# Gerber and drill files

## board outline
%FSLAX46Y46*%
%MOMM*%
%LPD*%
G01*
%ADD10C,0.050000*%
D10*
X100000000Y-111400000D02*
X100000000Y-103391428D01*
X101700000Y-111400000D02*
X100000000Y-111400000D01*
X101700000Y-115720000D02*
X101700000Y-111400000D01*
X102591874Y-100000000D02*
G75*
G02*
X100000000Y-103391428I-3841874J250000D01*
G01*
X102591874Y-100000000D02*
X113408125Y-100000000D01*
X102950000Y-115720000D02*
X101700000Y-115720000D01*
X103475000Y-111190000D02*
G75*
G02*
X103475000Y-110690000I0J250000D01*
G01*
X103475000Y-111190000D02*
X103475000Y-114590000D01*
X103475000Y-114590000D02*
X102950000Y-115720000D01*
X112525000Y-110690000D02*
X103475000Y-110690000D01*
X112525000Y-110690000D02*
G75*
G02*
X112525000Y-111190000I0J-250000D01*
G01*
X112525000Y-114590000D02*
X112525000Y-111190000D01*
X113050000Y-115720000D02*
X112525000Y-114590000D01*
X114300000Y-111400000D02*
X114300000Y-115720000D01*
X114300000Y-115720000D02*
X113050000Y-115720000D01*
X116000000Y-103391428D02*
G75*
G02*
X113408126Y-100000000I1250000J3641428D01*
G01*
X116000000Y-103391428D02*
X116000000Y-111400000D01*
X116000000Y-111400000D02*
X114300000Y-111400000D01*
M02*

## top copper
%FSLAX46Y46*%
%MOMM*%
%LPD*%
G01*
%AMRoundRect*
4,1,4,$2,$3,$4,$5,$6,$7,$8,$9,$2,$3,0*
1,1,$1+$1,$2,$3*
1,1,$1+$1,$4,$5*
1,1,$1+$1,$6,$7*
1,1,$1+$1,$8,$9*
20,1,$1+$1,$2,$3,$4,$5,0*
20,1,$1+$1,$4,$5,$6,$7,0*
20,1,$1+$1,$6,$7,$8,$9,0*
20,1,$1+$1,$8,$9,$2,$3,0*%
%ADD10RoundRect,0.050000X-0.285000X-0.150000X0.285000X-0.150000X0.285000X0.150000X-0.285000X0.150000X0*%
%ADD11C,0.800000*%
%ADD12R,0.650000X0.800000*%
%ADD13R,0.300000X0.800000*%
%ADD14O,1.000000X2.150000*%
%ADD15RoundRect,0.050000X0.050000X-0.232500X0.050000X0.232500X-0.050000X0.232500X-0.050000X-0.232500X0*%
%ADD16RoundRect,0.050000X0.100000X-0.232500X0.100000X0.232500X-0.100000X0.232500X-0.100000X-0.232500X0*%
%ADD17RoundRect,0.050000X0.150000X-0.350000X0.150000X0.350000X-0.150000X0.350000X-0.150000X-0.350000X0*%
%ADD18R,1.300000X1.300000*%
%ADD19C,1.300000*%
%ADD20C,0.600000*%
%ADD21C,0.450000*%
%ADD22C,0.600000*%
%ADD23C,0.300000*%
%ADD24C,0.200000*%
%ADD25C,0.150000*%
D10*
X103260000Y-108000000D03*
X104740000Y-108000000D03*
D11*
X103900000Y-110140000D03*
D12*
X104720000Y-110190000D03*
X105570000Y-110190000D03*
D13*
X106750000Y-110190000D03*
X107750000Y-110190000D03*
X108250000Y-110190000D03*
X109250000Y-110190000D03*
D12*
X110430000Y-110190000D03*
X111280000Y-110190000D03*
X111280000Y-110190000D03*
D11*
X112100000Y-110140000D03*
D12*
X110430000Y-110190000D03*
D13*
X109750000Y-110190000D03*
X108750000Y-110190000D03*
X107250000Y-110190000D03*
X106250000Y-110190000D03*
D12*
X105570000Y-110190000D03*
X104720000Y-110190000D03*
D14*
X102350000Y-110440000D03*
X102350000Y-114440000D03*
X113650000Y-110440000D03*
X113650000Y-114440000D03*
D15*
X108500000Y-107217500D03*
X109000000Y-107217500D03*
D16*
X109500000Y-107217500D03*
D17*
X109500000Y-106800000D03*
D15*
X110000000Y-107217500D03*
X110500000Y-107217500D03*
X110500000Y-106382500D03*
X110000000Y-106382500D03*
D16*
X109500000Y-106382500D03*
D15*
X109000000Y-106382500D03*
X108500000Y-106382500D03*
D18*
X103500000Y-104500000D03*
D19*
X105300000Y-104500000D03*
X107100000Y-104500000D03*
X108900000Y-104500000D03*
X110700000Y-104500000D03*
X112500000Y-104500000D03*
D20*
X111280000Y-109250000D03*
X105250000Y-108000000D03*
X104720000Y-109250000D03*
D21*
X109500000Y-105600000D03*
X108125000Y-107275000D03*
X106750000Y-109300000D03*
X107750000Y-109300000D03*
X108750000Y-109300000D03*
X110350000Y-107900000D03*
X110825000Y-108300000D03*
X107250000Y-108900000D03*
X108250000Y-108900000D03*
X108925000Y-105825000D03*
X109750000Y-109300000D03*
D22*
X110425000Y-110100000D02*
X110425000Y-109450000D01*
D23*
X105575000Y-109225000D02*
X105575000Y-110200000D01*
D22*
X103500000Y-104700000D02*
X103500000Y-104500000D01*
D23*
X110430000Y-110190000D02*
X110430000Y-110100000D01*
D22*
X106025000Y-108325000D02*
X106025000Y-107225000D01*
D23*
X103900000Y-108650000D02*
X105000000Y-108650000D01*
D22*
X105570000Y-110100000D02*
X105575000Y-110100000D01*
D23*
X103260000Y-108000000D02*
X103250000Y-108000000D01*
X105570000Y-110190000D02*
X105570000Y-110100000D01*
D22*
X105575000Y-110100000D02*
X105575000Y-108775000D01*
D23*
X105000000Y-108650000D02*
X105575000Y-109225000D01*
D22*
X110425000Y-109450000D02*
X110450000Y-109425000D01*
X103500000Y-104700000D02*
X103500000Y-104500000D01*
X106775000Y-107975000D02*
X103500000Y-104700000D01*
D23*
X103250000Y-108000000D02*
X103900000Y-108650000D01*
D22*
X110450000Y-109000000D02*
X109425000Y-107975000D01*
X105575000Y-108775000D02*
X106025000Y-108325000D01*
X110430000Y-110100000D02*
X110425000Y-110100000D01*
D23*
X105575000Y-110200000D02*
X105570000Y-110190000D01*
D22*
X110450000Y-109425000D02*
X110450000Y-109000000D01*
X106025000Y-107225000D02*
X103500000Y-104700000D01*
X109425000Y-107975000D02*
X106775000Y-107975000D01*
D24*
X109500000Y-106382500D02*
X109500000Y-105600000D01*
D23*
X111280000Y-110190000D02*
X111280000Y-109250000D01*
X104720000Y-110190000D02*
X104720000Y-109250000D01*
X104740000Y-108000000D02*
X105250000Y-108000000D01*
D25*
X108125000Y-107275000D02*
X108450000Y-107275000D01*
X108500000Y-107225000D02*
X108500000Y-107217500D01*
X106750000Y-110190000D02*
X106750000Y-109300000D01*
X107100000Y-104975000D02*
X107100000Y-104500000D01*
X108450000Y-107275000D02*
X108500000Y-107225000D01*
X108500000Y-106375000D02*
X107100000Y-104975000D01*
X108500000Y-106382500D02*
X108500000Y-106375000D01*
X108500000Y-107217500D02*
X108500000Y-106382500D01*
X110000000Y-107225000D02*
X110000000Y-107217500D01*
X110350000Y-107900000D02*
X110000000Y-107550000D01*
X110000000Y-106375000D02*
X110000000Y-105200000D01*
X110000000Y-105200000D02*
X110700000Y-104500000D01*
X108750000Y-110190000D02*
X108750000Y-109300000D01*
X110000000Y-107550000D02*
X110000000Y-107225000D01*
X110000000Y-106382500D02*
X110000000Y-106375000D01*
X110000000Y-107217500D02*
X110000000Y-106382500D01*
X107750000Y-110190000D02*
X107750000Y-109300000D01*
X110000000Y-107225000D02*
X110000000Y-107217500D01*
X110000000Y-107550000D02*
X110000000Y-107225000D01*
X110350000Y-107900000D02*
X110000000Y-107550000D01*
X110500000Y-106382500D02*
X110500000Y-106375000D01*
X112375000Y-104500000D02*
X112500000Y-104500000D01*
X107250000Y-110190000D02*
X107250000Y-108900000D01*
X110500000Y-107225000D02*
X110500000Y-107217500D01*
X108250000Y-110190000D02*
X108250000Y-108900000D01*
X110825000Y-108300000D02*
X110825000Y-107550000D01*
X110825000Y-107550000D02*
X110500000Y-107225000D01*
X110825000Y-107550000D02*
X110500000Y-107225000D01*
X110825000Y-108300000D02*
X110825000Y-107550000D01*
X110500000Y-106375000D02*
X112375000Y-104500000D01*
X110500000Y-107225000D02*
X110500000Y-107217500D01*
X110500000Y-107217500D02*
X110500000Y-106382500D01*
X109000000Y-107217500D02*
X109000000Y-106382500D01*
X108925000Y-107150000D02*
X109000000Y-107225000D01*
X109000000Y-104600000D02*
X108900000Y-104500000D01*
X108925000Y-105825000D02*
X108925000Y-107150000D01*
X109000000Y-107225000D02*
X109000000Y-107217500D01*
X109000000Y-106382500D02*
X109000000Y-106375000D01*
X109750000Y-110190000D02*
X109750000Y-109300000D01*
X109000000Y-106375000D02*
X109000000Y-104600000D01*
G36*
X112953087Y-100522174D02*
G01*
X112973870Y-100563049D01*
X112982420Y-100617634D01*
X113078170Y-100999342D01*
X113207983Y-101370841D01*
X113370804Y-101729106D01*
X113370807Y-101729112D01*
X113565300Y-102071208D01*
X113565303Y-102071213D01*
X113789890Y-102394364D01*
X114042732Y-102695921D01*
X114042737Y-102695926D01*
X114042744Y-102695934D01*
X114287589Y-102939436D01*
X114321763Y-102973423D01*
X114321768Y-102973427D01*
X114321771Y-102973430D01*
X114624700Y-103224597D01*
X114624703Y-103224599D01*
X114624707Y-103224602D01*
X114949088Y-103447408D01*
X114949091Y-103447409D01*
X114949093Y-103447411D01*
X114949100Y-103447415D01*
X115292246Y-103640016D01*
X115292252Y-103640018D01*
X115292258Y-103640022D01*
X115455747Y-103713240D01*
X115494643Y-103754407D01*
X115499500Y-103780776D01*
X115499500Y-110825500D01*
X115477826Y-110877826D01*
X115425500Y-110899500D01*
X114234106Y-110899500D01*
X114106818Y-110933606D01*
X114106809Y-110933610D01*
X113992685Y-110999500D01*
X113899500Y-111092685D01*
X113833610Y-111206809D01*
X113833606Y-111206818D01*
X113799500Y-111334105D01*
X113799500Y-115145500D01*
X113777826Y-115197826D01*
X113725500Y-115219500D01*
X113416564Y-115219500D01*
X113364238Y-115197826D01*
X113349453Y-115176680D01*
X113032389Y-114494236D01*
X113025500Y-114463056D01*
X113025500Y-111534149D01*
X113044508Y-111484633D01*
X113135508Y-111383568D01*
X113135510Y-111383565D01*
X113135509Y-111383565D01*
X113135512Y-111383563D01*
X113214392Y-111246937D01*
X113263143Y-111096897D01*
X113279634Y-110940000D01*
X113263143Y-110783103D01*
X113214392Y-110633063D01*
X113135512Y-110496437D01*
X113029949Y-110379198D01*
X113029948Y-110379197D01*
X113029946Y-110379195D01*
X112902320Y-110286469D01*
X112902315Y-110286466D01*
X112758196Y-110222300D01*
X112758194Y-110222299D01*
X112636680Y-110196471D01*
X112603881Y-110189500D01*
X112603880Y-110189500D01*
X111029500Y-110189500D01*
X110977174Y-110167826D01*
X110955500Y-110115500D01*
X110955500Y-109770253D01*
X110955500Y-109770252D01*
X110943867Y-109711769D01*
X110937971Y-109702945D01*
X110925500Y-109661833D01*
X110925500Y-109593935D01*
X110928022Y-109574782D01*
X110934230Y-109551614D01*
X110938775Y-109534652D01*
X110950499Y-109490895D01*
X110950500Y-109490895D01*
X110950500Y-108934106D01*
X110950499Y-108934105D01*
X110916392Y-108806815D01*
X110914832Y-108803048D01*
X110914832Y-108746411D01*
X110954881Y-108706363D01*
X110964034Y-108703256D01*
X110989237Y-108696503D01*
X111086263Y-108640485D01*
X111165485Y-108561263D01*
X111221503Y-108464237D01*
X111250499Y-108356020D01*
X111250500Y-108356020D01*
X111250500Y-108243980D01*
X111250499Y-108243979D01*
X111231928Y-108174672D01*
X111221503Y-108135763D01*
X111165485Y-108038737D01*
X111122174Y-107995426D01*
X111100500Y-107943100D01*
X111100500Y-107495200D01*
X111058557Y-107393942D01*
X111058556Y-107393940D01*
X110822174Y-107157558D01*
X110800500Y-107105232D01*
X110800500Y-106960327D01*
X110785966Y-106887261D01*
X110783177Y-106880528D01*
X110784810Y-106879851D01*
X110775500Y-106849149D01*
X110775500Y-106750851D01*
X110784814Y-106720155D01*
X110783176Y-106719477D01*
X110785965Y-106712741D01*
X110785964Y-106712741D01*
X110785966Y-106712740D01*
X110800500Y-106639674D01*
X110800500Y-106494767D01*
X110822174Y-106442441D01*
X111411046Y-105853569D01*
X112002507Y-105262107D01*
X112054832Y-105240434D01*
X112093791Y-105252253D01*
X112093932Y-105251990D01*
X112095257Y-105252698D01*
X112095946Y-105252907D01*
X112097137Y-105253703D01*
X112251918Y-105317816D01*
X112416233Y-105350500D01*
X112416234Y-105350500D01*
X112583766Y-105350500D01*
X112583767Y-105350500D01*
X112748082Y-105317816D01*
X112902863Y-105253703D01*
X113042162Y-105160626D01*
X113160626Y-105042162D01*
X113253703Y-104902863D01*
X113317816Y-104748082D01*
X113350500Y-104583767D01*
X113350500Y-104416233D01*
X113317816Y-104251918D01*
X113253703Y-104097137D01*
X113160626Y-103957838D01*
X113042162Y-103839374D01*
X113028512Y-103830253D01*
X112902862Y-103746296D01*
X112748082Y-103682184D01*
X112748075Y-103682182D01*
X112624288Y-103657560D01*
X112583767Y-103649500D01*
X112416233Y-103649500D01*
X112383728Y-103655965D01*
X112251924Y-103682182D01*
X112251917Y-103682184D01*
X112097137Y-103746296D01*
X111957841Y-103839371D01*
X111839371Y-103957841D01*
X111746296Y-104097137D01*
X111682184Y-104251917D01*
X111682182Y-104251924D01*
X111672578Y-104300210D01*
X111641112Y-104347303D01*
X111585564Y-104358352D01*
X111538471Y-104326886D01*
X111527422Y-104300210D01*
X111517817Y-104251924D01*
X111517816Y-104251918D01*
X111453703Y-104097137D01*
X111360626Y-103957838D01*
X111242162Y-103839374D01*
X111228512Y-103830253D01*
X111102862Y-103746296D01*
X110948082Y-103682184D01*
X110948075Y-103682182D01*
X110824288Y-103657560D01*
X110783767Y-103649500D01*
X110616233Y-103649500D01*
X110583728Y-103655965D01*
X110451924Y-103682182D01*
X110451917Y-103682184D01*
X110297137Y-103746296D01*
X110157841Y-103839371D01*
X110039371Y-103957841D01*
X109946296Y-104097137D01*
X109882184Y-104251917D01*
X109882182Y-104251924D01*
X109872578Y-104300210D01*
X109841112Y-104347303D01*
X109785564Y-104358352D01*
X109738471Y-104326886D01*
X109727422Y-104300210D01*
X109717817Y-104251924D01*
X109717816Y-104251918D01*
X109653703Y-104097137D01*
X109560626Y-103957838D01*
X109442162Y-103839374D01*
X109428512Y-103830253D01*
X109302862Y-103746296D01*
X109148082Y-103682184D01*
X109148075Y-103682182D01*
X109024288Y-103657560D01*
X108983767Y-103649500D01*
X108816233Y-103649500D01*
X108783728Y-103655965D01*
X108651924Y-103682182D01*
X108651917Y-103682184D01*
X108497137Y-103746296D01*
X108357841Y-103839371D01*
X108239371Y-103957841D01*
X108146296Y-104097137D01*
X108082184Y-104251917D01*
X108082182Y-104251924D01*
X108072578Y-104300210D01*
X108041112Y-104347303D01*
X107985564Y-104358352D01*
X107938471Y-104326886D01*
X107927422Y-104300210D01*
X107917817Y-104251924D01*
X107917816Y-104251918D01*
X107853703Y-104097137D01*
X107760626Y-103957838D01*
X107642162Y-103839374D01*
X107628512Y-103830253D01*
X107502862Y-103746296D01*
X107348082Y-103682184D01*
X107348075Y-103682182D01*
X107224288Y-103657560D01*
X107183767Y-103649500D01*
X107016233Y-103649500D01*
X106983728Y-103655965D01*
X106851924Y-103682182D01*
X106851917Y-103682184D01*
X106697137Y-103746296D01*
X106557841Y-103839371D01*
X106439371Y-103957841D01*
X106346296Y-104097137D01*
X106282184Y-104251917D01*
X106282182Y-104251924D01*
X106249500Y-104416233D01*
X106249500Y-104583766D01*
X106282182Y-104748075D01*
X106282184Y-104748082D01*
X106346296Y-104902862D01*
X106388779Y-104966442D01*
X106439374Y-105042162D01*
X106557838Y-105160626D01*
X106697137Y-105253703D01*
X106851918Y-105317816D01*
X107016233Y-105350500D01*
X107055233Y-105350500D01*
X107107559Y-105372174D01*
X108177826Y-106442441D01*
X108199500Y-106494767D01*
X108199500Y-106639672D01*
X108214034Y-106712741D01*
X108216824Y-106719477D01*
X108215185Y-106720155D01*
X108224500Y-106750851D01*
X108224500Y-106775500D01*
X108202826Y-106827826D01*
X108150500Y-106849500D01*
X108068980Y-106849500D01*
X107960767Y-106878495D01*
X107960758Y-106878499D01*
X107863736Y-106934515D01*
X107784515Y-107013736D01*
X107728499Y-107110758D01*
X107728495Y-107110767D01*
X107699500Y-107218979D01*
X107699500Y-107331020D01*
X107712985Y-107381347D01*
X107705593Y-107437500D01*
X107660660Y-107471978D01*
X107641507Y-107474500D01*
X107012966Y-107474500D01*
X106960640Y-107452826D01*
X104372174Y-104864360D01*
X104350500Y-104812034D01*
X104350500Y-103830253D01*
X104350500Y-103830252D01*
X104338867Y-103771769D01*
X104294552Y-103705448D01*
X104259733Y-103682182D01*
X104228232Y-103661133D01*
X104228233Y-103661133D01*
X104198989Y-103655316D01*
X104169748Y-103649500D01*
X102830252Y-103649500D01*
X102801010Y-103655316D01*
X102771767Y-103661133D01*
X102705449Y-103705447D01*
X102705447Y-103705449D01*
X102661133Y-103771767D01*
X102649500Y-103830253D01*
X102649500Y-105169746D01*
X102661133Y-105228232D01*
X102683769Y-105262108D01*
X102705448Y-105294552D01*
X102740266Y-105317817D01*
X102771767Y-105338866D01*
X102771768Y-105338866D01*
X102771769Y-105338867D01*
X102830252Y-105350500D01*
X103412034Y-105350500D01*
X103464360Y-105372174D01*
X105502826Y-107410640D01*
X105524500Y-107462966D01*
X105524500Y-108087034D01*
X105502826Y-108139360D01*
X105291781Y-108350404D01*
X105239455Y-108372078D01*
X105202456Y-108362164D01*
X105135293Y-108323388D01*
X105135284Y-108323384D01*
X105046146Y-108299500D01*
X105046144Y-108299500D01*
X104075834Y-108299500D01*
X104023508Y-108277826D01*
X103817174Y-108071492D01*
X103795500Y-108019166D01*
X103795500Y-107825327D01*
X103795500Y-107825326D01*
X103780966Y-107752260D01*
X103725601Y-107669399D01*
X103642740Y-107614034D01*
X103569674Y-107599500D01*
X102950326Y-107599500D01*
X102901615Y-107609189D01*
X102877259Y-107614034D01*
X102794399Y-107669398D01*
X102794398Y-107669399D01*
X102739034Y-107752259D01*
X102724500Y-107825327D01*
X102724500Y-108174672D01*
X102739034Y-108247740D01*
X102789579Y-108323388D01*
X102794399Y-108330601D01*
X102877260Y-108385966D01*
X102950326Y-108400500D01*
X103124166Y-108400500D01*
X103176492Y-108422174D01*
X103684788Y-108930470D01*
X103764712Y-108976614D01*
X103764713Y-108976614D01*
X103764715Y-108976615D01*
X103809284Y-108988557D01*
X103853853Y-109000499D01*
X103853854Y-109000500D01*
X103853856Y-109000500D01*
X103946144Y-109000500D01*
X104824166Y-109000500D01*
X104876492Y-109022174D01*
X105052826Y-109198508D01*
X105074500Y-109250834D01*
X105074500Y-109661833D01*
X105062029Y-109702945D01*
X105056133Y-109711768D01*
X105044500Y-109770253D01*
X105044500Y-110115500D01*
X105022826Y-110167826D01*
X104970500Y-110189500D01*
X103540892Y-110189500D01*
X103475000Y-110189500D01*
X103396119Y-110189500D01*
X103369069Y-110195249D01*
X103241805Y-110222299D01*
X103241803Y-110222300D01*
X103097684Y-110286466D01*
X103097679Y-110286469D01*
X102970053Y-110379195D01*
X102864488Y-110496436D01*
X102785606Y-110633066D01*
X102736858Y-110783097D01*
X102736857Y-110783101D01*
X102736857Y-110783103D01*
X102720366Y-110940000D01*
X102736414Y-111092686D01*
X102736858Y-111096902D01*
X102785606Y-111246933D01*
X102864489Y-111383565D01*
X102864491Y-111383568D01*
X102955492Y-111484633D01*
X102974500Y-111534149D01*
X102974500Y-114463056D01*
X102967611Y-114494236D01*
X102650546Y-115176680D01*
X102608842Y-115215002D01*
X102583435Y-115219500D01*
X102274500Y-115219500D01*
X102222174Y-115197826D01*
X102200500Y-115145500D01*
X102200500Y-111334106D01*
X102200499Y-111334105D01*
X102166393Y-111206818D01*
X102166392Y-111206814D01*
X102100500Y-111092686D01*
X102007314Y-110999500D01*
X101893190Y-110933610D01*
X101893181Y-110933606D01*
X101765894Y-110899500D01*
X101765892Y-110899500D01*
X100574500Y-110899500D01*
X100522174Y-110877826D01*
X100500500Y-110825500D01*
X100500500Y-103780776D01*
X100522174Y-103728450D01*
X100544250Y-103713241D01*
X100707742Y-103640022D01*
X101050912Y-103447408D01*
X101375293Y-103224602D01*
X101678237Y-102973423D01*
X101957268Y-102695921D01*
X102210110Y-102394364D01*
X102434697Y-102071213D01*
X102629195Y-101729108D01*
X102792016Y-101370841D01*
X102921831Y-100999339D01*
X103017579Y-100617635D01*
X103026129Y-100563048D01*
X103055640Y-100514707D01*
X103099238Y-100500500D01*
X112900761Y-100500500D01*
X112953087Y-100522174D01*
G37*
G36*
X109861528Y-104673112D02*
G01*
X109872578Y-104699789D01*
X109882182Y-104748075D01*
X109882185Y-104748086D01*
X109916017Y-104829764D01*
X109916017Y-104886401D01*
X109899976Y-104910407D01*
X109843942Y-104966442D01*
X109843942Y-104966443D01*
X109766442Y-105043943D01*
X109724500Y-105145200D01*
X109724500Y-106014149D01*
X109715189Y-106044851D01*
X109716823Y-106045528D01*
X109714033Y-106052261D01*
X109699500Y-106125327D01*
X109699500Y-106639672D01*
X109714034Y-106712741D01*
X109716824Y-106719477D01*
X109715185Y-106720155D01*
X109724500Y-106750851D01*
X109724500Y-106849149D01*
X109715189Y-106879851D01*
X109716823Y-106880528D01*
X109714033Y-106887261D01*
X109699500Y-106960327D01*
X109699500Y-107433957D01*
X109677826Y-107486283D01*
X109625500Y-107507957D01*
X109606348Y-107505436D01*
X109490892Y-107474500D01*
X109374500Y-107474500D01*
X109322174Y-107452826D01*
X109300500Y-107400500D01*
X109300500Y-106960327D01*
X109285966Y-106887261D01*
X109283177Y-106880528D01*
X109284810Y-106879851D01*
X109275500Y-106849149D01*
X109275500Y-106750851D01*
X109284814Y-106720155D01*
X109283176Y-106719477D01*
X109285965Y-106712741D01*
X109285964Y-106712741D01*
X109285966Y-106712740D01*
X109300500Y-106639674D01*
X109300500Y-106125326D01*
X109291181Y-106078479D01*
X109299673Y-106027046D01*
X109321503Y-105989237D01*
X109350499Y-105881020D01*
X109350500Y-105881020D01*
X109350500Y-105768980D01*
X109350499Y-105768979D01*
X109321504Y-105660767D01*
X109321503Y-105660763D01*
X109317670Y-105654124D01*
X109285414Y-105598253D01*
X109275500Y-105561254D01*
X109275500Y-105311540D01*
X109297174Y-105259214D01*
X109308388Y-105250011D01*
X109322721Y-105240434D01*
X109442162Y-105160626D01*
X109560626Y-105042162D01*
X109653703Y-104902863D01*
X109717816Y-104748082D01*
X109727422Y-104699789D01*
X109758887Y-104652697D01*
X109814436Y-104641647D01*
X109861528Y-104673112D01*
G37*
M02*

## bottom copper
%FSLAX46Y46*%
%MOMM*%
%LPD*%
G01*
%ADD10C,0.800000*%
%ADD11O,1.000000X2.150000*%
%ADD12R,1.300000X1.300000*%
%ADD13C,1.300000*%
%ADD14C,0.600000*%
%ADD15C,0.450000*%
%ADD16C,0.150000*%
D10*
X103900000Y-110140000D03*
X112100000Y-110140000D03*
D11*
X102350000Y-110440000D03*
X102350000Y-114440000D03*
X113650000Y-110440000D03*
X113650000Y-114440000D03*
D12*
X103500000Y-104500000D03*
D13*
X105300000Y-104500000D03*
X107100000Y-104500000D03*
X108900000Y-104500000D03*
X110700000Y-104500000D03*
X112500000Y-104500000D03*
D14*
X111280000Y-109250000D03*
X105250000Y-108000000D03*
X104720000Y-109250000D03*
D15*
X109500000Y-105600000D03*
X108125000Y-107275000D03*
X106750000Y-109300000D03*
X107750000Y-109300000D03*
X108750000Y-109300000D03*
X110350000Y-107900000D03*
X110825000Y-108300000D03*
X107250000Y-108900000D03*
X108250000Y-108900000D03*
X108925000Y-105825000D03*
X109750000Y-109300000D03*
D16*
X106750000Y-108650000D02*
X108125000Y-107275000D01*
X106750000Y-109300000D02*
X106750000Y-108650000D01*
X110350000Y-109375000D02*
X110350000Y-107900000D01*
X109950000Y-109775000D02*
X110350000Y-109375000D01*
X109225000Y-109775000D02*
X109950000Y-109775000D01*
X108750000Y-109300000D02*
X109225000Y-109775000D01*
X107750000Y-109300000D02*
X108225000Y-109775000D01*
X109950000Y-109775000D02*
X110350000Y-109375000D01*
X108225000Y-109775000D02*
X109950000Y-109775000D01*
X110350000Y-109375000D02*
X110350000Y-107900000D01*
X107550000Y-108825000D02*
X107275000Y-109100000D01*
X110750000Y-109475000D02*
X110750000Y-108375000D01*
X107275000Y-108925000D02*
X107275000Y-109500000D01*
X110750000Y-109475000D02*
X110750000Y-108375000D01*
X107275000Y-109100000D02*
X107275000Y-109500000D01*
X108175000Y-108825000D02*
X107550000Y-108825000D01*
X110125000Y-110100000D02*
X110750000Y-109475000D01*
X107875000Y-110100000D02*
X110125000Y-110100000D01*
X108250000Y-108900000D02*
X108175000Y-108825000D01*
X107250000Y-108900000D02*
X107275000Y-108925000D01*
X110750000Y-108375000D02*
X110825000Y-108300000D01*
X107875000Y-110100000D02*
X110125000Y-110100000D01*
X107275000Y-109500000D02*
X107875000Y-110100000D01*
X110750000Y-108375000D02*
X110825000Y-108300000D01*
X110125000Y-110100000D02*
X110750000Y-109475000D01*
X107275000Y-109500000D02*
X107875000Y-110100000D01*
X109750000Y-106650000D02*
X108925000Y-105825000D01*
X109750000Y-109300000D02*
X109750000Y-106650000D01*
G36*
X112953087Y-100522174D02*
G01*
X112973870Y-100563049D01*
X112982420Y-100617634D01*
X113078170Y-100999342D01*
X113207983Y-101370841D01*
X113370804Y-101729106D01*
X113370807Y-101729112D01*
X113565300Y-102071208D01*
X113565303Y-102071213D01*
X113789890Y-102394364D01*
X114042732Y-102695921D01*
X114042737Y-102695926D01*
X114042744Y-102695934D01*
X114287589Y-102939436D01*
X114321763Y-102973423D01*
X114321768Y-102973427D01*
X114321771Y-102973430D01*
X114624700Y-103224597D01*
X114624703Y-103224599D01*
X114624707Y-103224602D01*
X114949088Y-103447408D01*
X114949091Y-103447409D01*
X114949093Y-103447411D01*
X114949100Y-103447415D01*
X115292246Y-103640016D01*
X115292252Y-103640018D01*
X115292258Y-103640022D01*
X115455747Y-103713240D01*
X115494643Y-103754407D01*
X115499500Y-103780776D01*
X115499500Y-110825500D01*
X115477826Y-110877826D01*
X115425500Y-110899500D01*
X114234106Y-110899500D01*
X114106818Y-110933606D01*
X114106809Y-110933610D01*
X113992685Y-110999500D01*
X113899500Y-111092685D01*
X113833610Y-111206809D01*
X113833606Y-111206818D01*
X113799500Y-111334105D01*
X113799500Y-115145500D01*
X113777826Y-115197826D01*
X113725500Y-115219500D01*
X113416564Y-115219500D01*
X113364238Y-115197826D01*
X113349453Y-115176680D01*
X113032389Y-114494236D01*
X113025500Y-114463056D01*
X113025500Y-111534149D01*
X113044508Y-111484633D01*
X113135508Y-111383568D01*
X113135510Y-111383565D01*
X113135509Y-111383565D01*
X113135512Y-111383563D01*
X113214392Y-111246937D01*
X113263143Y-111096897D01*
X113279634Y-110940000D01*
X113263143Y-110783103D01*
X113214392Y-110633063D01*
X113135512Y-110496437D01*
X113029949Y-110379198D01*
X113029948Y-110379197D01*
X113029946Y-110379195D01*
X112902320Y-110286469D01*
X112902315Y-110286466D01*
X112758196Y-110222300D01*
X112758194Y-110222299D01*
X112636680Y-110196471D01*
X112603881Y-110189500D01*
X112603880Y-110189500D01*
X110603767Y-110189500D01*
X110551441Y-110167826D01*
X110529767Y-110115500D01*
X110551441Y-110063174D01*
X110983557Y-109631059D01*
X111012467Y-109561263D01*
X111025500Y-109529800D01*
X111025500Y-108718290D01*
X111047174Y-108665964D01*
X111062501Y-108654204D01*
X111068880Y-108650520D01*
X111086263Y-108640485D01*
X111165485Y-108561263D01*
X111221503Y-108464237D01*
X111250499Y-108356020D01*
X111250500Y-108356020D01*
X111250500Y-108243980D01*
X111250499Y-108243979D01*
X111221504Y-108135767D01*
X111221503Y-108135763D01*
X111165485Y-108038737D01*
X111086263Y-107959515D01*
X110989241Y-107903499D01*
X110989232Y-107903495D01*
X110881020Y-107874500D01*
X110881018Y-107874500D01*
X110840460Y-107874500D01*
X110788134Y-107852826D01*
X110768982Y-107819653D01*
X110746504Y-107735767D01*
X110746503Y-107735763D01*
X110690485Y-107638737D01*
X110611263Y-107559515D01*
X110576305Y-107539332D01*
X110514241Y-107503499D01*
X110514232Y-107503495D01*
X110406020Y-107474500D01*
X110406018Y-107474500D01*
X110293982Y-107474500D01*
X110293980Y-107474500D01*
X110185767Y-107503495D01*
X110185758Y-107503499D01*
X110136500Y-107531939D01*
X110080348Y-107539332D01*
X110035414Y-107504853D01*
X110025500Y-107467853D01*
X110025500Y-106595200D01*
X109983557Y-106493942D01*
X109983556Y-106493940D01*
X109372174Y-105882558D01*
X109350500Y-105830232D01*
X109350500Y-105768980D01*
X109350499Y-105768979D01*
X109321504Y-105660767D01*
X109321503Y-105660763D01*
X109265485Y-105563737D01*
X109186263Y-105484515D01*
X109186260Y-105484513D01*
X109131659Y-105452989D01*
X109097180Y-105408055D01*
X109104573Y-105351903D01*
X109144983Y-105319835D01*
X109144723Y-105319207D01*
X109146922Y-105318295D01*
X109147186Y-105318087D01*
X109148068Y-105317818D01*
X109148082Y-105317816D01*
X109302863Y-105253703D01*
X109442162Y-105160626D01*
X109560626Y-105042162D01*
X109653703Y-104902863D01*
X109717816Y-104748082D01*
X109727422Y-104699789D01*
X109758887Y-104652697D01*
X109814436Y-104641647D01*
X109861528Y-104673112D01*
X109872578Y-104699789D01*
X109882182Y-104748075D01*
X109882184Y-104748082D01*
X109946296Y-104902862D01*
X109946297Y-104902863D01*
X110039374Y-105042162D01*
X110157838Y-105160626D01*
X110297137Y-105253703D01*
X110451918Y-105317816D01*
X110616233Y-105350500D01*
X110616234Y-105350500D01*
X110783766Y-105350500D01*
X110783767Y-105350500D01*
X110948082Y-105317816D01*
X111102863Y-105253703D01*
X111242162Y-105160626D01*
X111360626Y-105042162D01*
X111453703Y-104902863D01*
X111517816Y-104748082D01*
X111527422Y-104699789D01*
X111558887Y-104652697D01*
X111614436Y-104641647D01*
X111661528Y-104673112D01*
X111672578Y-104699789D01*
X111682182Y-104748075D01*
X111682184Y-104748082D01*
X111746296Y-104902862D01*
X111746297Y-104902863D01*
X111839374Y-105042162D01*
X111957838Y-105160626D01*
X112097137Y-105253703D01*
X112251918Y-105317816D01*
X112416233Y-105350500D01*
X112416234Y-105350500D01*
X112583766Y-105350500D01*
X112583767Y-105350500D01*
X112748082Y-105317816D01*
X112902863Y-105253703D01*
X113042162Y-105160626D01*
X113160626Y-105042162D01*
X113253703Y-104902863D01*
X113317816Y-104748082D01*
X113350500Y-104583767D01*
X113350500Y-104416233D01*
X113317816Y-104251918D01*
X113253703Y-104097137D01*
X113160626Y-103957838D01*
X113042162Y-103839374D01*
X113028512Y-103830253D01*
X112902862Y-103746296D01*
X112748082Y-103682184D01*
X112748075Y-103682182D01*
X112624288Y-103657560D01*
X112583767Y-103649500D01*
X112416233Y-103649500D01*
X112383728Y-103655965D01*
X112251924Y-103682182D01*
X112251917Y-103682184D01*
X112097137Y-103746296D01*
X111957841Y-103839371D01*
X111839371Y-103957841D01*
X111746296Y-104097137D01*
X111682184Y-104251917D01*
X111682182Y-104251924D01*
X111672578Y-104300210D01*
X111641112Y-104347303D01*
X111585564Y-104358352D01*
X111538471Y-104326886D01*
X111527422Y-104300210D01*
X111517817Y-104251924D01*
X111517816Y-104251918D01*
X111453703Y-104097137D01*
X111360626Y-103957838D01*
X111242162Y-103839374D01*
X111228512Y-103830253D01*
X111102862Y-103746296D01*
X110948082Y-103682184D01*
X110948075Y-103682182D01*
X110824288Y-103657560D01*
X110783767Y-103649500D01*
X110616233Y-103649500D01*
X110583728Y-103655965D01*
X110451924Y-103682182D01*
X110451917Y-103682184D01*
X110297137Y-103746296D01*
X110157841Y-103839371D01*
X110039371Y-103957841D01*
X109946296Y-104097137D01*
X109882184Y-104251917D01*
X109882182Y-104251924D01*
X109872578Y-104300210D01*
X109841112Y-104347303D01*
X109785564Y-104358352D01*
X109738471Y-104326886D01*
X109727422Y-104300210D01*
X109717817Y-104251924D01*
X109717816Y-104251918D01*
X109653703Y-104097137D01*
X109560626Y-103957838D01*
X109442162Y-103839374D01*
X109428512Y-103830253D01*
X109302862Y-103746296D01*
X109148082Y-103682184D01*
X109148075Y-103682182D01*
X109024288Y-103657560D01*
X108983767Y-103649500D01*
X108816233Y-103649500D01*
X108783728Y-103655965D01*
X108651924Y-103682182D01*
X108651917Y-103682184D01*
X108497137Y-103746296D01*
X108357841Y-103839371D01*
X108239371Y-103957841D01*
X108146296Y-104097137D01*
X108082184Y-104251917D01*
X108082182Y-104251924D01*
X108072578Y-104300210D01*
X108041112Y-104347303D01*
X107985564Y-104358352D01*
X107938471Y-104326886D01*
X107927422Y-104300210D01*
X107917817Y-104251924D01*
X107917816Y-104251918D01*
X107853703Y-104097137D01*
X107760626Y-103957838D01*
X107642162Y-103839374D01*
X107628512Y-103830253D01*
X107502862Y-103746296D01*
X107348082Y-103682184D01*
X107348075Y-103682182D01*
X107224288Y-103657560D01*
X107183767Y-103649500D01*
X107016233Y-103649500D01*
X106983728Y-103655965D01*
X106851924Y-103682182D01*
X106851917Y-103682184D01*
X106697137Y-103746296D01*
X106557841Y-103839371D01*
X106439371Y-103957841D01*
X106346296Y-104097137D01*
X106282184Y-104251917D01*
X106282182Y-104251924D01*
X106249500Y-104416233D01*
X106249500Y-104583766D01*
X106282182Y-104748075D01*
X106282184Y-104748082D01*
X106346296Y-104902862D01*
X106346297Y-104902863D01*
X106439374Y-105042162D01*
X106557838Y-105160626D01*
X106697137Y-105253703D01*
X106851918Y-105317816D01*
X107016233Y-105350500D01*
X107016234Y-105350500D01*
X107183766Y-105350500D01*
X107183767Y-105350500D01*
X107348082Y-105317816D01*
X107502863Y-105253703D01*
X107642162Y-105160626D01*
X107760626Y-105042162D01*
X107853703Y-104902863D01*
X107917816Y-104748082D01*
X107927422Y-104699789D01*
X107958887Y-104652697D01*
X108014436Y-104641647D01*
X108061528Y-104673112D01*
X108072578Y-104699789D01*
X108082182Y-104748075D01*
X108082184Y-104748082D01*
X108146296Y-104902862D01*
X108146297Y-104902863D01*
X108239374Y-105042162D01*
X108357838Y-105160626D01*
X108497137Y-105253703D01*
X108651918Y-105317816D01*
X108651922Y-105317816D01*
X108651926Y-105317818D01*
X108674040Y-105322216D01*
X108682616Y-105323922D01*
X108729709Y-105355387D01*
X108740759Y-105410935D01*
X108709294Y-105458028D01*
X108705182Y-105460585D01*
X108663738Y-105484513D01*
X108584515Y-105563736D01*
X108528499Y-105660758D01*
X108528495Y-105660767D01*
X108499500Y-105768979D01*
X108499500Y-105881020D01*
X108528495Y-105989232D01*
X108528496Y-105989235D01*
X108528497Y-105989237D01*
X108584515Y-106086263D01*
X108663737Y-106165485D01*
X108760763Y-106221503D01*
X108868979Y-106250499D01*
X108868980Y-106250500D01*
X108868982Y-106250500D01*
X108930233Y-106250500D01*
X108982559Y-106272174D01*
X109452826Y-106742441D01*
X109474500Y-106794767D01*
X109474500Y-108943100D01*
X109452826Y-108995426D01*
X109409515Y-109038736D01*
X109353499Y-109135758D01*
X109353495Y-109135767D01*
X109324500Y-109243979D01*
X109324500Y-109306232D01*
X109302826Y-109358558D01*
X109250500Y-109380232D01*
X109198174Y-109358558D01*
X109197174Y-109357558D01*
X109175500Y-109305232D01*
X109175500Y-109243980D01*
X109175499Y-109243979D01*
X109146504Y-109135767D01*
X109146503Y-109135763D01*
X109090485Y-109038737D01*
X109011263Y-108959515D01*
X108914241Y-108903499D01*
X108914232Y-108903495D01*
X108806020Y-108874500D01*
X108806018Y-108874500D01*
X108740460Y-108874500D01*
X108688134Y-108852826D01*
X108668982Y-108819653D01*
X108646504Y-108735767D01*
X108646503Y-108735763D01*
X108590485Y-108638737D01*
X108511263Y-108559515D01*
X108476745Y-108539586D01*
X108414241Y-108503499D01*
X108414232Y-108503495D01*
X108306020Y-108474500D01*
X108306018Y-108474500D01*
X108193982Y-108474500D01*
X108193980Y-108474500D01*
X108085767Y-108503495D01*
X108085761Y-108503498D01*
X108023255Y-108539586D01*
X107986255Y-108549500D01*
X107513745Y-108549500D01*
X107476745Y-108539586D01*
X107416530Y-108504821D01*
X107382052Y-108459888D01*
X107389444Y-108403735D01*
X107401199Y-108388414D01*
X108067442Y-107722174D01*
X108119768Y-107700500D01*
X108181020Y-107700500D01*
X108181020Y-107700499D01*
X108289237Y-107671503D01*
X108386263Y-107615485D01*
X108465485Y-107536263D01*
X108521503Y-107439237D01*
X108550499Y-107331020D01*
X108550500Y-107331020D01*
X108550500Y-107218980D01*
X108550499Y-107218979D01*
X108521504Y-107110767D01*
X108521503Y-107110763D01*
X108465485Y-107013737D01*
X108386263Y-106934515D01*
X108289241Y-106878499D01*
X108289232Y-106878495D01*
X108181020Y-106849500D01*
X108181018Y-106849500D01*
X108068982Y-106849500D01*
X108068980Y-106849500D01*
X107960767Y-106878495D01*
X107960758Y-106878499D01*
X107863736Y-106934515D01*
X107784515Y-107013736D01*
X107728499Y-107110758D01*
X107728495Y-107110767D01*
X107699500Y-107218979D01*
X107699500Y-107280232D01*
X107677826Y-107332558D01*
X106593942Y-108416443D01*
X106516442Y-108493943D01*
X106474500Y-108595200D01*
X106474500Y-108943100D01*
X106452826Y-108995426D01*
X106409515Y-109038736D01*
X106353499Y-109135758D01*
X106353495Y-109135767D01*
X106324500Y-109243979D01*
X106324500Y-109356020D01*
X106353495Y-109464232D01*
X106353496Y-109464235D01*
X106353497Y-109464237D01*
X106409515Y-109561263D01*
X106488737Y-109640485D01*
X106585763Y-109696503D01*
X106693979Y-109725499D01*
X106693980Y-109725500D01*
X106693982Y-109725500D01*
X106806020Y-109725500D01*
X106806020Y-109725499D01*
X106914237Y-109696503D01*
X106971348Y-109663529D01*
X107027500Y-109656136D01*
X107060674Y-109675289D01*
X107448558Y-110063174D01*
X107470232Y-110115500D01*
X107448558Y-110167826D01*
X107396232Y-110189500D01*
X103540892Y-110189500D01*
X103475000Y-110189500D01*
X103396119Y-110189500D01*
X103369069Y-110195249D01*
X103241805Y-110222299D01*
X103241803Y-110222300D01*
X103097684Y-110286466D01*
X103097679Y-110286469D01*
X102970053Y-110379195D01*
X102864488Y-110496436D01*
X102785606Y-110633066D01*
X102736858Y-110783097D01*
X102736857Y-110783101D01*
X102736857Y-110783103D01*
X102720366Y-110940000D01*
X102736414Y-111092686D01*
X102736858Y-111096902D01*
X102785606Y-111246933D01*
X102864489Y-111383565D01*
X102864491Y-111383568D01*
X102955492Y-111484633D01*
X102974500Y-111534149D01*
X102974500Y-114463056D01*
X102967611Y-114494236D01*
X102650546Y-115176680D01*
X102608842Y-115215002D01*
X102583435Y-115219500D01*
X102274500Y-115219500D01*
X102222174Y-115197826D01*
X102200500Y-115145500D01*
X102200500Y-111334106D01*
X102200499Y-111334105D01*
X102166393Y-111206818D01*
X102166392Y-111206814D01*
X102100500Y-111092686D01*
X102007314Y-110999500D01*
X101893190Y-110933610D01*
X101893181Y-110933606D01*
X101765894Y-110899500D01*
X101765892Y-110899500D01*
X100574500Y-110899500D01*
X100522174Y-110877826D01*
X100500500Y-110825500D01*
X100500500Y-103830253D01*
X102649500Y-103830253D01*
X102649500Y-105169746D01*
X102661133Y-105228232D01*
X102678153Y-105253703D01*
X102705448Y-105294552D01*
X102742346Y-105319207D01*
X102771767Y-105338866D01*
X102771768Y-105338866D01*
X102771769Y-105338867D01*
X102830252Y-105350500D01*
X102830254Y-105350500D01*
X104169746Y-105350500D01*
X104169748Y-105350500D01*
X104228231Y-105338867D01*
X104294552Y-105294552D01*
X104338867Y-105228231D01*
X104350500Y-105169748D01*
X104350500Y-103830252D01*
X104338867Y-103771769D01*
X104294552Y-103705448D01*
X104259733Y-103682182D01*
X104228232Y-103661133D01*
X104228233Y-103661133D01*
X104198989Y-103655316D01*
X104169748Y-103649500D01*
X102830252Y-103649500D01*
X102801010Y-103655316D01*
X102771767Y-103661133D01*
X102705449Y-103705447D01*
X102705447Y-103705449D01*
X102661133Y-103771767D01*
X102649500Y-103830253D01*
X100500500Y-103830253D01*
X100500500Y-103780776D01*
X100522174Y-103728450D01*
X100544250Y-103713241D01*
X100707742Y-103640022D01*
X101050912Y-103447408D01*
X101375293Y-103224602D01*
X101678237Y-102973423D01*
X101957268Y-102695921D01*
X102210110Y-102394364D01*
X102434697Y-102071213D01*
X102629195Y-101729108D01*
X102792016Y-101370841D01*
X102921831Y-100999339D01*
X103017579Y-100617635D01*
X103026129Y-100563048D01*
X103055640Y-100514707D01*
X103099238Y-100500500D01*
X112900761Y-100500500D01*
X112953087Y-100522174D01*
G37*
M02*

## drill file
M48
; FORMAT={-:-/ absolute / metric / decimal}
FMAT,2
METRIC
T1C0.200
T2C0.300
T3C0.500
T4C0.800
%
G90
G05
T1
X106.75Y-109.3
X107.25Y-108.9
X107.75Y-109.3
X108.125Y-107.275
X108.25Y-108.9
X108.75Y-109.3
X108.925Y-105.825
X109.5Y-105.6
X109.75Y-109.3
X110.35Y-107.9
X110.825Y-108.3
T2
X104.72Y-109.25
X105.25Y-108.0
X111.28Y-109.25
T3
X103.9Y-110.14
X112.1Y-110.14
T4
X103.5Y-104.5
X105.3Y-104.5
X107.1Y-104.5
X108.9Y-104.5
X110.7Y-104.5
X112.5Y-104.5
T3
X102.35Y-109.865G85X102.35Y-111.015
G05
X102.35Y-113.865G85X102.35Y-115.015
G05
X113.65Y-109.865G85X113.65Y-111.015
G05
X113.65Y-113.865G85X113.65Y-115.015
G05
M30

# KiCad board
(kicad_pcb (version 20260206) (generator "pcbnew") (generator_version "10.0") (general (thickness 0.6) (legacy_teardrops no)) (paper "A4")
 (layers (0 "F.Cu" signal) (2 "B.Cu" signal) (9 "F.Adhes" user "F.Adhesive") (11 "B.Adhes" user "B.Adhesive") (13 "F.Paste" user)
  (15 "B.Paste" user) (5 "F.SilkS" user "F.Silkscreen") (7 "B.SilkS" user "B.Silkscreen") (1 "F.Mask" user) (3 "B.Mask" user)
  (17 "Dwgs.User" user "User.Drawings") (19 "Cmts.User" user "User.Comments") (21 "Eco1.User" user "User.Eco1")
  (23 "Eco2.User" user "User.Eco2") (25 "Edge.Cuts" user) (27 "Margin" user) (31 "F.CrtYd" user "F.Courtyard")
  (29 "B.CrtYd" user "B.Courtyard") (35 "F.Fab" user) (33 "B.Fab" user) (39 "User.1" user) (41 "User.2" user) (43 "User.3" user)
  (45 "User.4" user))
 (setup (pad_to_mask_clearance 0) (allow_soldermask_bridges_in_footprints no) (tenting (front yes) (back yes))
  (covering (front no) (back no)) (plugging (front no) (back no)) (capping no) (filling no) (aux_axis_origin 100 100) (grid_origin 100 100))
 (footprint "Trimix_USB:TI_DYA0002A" (layer "F.Cu") (at 104 108)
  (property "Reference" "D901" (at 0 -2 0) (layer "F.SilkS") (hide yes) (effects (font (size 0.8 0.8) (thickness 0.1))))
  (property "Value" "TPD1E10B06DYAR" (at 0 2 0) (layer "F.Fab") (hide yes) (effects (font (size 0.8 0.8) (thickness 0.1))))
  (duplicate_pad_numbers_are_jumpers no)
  (pad "1" smd roundrect (at -0.74 0) (size 0.67 0.4) (layers "F.Cu" "F.Mask" "F.Paste") (roundrect_rratio 0.125) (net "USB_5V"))
  (pad "2" smd roundrect (at 0.74 0) (size 0.67 0.4) (layers "F.Cu" "F.Mask" "F.Paste") (roundrect_rratio 0.125) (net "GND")
   (zone_connect 2)))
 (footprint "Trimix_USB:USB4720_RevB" (layer "F.Cu") (at 108 110.14)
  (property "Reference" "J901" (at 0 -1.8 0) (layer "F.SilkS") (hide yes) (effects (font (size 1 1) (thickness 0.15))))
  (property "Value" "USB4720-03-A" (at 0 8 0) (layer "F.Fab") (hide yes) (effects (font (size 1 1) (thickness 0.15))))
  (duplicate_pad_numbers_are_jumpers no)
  (pad "A1" thru_hole circle (at -4.1 0) (size 0.8 0.8) (drill 0.5) (layers "*.Cu" "*.Mask") (remove_unused_layers no) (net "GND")
   (zone_connect 2))
  (pad "A1" smd rect (at -3.28 0.05) (size 0.65 0.8) (layers "F.Cu" "F.Mask" "F.Paste") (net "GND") (zone_connect 2))
  (pad "A4" smd rect (at -2.43 0.05) (size 0.65 0.8) (layers "F.Cu" "F.Mask" "F.Paste") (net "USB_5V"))
  (pad "A5" smd rect (at -1.25 0.05) (size 0.3 0.8) (layers "F.Cu" "F.Mask" "F.Paste") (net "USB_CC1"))
  (pad "A6" smd rect (at -0.25 0.05) (size 0.3 0.8) (layers "F.Cu" "F.Mask" "F.Paste") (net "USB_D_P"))
  (pad "A7" smd rect (at 0.25 0.05) (size 0.3 0.8) (layers "F.Cu" "F.Mask" "F.Paste") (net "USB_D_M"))
  (pad "A8" smd rect (at 1.25 0.05) (size 0.3 0.8) (layers "F.Cu" "F.Mask" "F.Paste") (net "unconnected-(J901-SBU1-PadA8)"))
  (pad "A9" smd rect (at 2.43 0.05) (size 0.65 0.8) (layers "F.Cu" "F.Mask" "F.Paste") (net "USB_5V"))
  (pad "A12" smd rect (at 3.28 0.05) (size 0.65 0.8) (layers "F.Cu" "F.Mask" "F.Paste") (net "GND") (zone_connect 2))
  (pad "B1" smd rect (at 3.28 0.05) (size 0.65 0.8) (layers "F.Cu" "F.Mask" "F.Paste") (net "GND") (zone_connect 2))
  (pad "B1" thru_hole circle (at 4.1 0) (size 0.8 0.8) (drill 0.5) (layers "*.Cu" "*.Mask") (remove_unused_layers no) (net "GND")
   (zone_connect 2))
  (pad "B4" smd rect (at 2.43 0.05) (size 0.65 0.8) (layers "F.Cu" "F.Mask" "F.Paste") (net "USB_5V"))
  (pad "B5" smd rect (at 1.75 0.05) (size 0.3 0.8) (layers "F.Cu" "F.Mask" "F.Paste") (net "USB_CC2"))
  (pad "B6" smd rect (at 0.75 0.05) (size 0.3 0.8) (layers "F.Cu" "F.Mask" "F.Paste") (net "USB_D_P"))
  (pad "B7" smd rect (at -0.75 0.05) (size 0.3 0.8) (layers "F.Cu" "F.Mask" "F.Paste") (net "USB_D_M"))
  (pad "B8" smd rect (at -1.75 0.05) (size 0.3 0.8) (layers "F.Cu" "F.Mask" "F.Paste") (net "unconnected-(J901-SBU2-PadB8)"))
  (pad "B9" smd rect (at -2.43 0.05) (size 0.65 0.8) (layers "F.Cu" "F.Mask" "F.Paste") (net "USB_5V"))
  (pad "B12" smd rect (at -3.28 0.05) (size 0.65 0.8) (layers "F.Cu" "F.Mask" "F.Paste") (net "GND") (zone_connect 2))
  (pad "SH" thru_hole oval (at -5.65 0.3) (size 1 2.15) (drill oval 0.5 1.65) (layers "*.Cu" "*.Mask") (remove_unused_layers no) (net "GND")
   (zone_connect 2))
  (pad "SH" thru_hole oval (at -5.65 4.3) (size 1 2.15) (drill oval 0.5 1.65) (layers "*.Cu" "*.Mask") (remove_unused_layers no) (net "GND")
   (zone_connect 2))
  (pad "SH" thru_hole oval (at 5.65 0.3) (size 1 2.15) (drill oval 0.5 1.65) (layers "*.Cu" "*.Mask") (remove_unused_layers no) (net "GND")
   (zone_connect 2))
  (pad "SH" thru_hole oval (at 5.65 4.3) (size 1 2.15) (drill oval 0.5 1.65) (layers "*.Cu" "*.Mask") (remove_unused_layers no) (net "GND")
   (zone_connect 2)))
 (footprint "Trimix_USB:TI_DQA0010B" (layer "F.Cu") (at 109.5 106.8 90)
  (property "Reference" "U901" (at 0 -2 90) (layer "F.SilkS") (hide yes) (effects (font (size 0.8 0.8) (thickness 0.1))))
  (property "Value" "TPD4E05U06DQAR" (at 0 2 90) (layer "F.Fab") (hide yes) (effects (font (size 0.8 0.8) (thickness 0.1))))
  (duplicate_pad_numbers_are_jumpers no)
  (pad "1" smd roundrect (at -0.4175 -1 90) (size 0.565 0.2) (layers "F.Cu" "F.Mask" "F.Paste") (roundrect_rratio 0.25) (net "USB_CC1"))
  (pad "2" smd roundrect (at -0.4175 -0.5 90) (size 0.565 0.2) (layers "F.Cu" "F.Mask" "F.Paste") (roundrect_rratio 0.25) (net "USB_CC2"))
  (pad "3" smd roundrect (at -0.4175 0 90) (size 0.565 0.3) (layers "F.Cu" "F.Mask" "F.Paste") (roundrect_rratio 0.1666666667) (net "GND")
   (zone_connect 2))
  (pad "3" smd roundrect (at 0 0 90) (size 0.8 0.4) (layers "F.Cu" "F.Mask") (roundrect_rratio 0.125) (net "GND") (zone_connect 2))
  (pad "4" smd roundrect (at -0.4175 0.5 90) (size 0.565 0.2) (layers "F.Cu" "F.Mask" "F.Paste") (roundrect_rratio 0.25) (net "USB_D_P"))
  (pad "5" smd roundrect (at -0.4175 1 90) (size 0.565 0.2) (layers "F.Cu" "F.Mask" "F.Paste") (roundrect_rratio 0.25) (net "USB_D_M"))
  (pad "6" smd roundrect (at 0.4175 1 90) (size 0.565 0.2) (layers "F.Cu" "F.Mask" "F.Paste") (roundrect_rratio 0.25) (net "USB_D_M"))
  (pad "7" smd roundrect (at 0.4175 0.5 90) (size 0.565 0.2) (layers "F.Cu" "F.Mask" "F.Paste") (roundrect_rratio 0.25) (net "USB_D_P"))
  (pad "8" smd roundrect (at 0.4175 0 90) (size 0.565 0.3) (layers "F.Cu" "F.Mask" "F.Paste") (roundrect_rratio 0.1666666667) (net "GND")
   (zone_connect 2))
  (pad "9" smd roundrect (at 0.4175 -0.5 90) (size 0.565 0.2) (layers "F.Cu" "F.Mask" "F.Paste") (roundrect_rratio 0.25) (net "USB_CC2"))
  (pad "10" smd roundrect (at 0.4175 -1 90) (size 0.565 0.2) (layers "F.Cu" "F.Mask" "F.Paste") (roundrect_rratio 0.25) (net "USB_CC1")))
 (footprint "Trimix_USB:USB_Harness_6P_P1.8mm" (layer "F.Cu") (at 108 104.5)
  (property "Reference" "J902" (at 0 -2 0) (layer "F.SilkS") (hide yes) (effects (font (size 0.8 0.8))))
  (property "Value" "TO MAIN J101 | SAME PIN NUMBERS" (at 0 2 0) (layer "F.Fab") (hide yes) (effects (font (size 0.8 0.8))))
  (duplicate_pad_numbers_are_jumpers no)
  (pad "1" thru_hole rect (at -4.5 0) (size 1.3 1.3) (drill 0.8) (layers "*.Cu" "*.Mask") (remove_unused_layers no) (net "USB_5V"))
  (pad "2" thru_hole circle (at -2.7 0) (size 1.3 1.3) (drill 0.8) (layers "*.Cu" "*.Mask") (remove_unused_layers no) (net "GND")
   (zone_connect 2))
  (pad "3" thru_hole circle (at -0.9 0) (size 1.3 1.3) (drill 0.8) (layers "*.Cu" "*.Mask") (remove_unused_layers no) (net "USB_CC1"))
  (pad "4" thru_hole circle (at 0.9 0) (size 1.3 1.3) (drill 0.8) (layers "*.Cu" "*.Mask") (remove_unused_layers no) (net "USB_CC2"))
  (pad "5" thru_hole circle (at 2.7 0) (size 1.3 1.3) (drill 0.8) (layers "*.Cu" "*.Mask") (remove_unused_layers no) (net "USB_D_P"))
  (pad "6" thru_hole circle (at 4.5 0) (size 1.3 1.3) (drill 0.8) (layers "*.Cu" "*.Mask") (remove_unused_layers no) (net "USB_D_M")))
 (gr_line (start 100 111.4) (end 100 103.391428) (stroke (width 0.05) (type default)) (layer "Edge.Cuts"))
 (gr_line (start 101.7 111.4) (end 100 111.4) (stroke (width 0.05) (type default)) (layer "Edge.Cuts"))
 (gr_line (start 101.7 115.72) (end 101.7 111.4) (stroke (width 0.05) (type default)) (layer "Edge.Cuts"))
 (gr_arc (start 102.591874 100) (mid 101.808961 102.087789) (end 100 103.391428) (stroke (width 0.05) (type default)) (layer "Edge.Cuts"))
 (gr_line (start 102.591874 100) (end 113.408125 100) (stroke (width 0.05) (type default)) (layer "Edge.Cuts"))
 (gr_line (start 102.95 115.72) (end 101.7 115.72) (stroke (width 0.05) (type default)) (layer "Edge.Cuts"))
 (gr_arc (start 103.475 111.19) (mid 103.225 110.94) (end 103.475 110.69) (stroke (width 0.05) (type default)) (layer "Edge.Cuts"))
 (gr_line (start 103.475 111.19) (end 103.475 114.59) (stroke (width 0.05) (type default)) (layer "Edge.Cuts"))
 (gr_line (start 103.475 114.59) (end 102.95 115.72) (stroke (width 0.05) (type default)) (layer "Edge.Cuts"))
 (gr_line (start 112.525 110.69) (end 103.475 110.69) (stroke (width 0.05) (type default)) (layer "Edge.Cuts"))
 (gr_arc (start 112.525 110.69) (mid 112.775 110.94) (end 112.525 111.19) (stroke (width 0.05) (type default)) (layer "Edge.Cuts"))
 (gr_line (start 112.525 114.59) (end 112.525 111.19) (stroke (width 0.05) (type default)) (layer "Edge.Cuts"))
 (gr_line (start 113.05 115.72) (end 112.525 114.59) (stroke (width 0.05) (type default)) (layer "Edge.Cuts"))
 (gr_line (start 114.3 111.4) (end 114.3 115.72) (stroke (width 0.05) (type default)) (layer "Edge.Cuts"))
 (gr_line (start 114.3 115.72) (end 113.05 115.72) (stroke (width 0.05) (type default)) (layer "Edge.Cuts"))
 (gr_arc (start 116 103.391428) (mid 114.191039 102.087789) (end 113.408125 100) (stroke (width 0.05) (type default)) (layer "Edge.Cuts"))
 (gr_line (start 116 103.391428) (end 116 111.4) (stroke (width 0.05) (type default)) (layer "Edge.Cuts"))
 (gr_line (start 116 111.4) (end 114.3 111.4) (stroke (width 0.05) (type default)) (layer "Edge.Cuts"))
 (segment (start 110.425 110.1) (end 110.425 109.45) (width 0.6) (layer "F.Cu") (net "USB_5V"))
 (segment (start 105.575 109.225) (end 105.575 110.2) (width 0.3) (layer "F.Cu") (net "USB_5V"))
 (segment (start 103.5 104.7) (end 103.5 104.5) (width 0.6) (layer "F.Cu") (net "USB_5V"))
 (segment (start 110.43 110.19) (end 110.43 110.1) (width 0.3) (layer "F.Cu") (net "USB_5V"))
 (segment (start 106.025 108.325) (end 106.025 107.225) (width 0.6) (layer "F.Cu") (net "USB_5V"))
 (segment (start 103.9 108.65) (end 105 108.65) (width 0.3) (layer "F.Cu") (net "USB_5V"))
 (segment (start 105.57 110.1) (end 105.575 110.1) (width 0.6) (layer "F.Cu") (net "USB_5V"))
 (segment (start 103.26 108) (end 103.25 108) (width 0.3) (layer "F.Cu") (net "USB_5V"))
 (segment (start 105.57 110.19) (end 105.57 110.1) (width 0.3) (layer "F.Cu") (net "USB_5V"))
 (segment (start 105.575 110.1) (end 105.575 108.775) (width 0.6) (layer "F.Cu") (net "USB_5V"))
 (segment (start 105 108.65) (end 105.575 109.225) (width 0.3) (layer "F.Cu") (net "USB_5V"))
 (segment (start 110.425 109.45) (end 110.45 109.425) (width 0.6) (layer "F.Cu") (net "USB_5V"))
 (segment (start 103.5 104.7) (end 103.5 104.5) (width 0.6) (layer "F.Cu") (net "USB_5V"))
 (segment (start 106.775 107.975) (end 103.5 104.7) (width 0.6) (layer "F.Cu") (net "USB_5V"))
 (segment (start 103.25 108) (end 103.9 108.65) (width 0.3) (layer "F.Cu") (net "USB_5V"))
 (segment (start 110.45 109) (end 109.425 107.975) (width 0.6) (layer "F.Cu") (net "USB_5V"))
 (segment (start 105.575 108.775) (end 106.025 108.325) (width 0.6) (layer "F.Cu") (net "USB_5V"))
 (segment (start 110.43 110.1) (end 110.425 110.1) (width 0.6) (layer "F.Cu") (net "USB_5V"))
 (segment (start 105.575 110.2) (end 105.57 110.19) (width 0.3) (layer "F.Cu") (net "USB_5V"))
 (segment (start 110.45 109.425) (end 110.45 109) (width 0.6) (layer "F.Cu") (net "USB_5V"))
 (segment (start 106.025 107.225) (end 103.5 104.7) (width 0.6) (layer "F.Cu") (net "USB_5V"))
 (segment (start 109.425 107.975) (end 106.775 107.975) (width 0.6) (layer "F.Cu") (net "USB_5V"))
 (segment (start 109.5 106.3825) (end 109.5 105.6) (width 0.2) (layer "F.Cu") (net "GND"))
 (segment (start 111.28 110.19) (end 111.28 109.25) (width 0.3) (layer "F.Cu") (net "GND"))
 (segment (start 104.72 110.19) (end 104.72 109.25) (width 0.3) (layer "F.Cu") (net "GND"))
 (segment (start 104.74 108) (end 105.25 108) (width 0.3) (layer "F.Cu") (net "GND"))
 (via (at 111.28 109.25) (size 0.6) (drill 0.3) (layers "F.Cu" "B.Cu") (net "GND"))
 (via (at 105.25 108) (size 0.6) (drill 0.3) (layers "F.Cu" "B.Cu") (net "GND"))
 (via (at 104.72 109.25) (size 0.6) (drill 0.3) (layers "F.Cu" "B.Cu") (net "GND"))
 (via (at 109.5 105.6) (size 0.45) (drill 0.2) (layers "F.Cu" "B.Cu") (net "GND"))
 (segment (start 108.125 107.275) (end 108.45 107.275) (width 0.15) (layer "F.Cu") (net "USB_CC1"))
 (segment (start 108.5 107.225) (end 108.5 107.2175) (width 0.15) (layer "F.Cu") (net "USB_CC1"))
 (segment (start 106.75 110.19) (end 106.75 109.3) (width 0.15) (layer "F.Cu") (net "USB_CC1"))
 (segment (start 107.1 104.975) (end 107.1 104.5) (width 0.15) (layer "F.Cu") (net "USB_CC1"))
 (segment (start 108.45 107.275) (end 108.5 107.225) (width 0.15) (layer "F.Cu") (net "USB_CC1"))
 (segment (start 108.5 106.375) (end 107.1 104.975) (width 0.15) (layer "F.Cu") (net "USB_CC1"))
 (segment (start 108.5 106.3825) (end 108.5 106.375) (width 0.15) (layer "F.Cu") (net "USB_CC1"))
 (segment (start 108.5 107.2175) (end 108.5 106.3825) (width 0.15) (layer "F.Cu") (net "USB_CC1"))
 (via (at 108.125 107.275) (size 0.45) (drill 0.2) (layers "F.Cu" "B.Cu") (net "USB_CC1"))
 (via (at 106.75 109.3) (size 0.45) (drill 0.2) (layers "F.Cu" "B.Cu") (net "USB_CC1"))
 (segment (start 106.75 108.65) (end 108.125 107.275) (width 0.15) (layer "B.Cu") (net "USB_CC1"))
 (segment (start 106.75 109.3) (end 106.75 108.65) (width 0.15) (layer "B.Cu") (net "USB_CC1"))
 (segment (start 110 107.225) (end 110 107.2175) (width 0.15) (layer "F.Cu") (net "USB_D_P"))
 (segment (start 110.35 107.9) (end 110 107.55) (width 0.15) (layer "F.Cu") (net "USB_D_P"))
 (segment (start 110 106.375) (end 110 105.2) (width 0.15) (layer "F.Cu") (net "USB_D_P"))
 (segment (start 110 105.2) (end 110.7 104.5) (width 0.15) (layer "F.Cu") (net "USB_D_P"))
 (segment (start 108.75 110.19) (end 108.75 109.3) (width 0.15) (layer "F.Cu") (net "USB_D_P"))
 (segment (start 110 107.55) (end 110 107.225) (width 0.15) (layer "F.Cu") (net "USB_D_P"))
 (segment (start 110 106.3825) (end 110 106.375) (width 0.15) (layer "F.Cu") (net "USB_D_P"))
 (segment (start 110 107.2175) (end 110 106.3825) (width 0.15) (layer "F.Cu") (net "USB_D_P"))
 (segment (start 107.75 110.19) (end 107.75 109.3) (width 0.15) (layer "F.Cu") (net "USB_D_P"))
 (segment (start 110 107.225) (end 110 107.2175) (width 0.15) (layer "F.Cu") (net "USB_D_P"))
 (segment (start 110 107.55) (end 110 107.225) (width 0.15) (layer "F.Cu") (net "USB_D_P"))
 (segment (start 110.35 107.9) (end 110 107.55) (width 0.15) (layer "F.Cu") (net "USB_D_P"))
 (via (at 107.75 109.3) (size 0.45) (drill 0.2) (layers "F.Cu" "B.Cu") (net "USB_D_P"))
 (via (at 108.75 109.3) (size 0.45) (drill 0.2) (layers "F.Cu" "B.Cu") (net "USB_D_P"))
 (via (at 110.35 107.9) (size 0.45) (drill 0.2) (layers "F.Cu" "B.Cu") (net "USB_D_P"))
 (segment (start 110.35 109.375) (end 110.35 107.9) (width 0.15) (layer "B.Cu") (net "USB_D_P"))
 (segment (start 109.95 109.775) (end 110.35 109.375) (width 0.15) (layer "B.Cu") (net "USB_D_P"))
 (segment (start 109.225 109.775) (end 109.95 109.775) (width 0.15) (layer "B.Cu") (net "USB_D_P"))
 (segment (start 108.75 109.3) (end 109.225 109.775) (width 0.15) (layer "B.Cu") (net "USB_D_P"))
 (segment (start 107.75 109.3) (end 108.225 109.775) (width 0.15) (layer "B.Cu") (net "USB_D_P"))
 (segment (start 109.95 109.775) (end 110.35 109.375) (width 0.15) (layer "B.Cu") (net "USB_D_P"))
 (segment (start 108.225 109.775) (end 109.95 109.775) (width 0.15) (layer "B.Cu") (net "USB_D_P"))
 (segment (start 110.35 109.375) (end 110.35 107.9) (width 0.15) (layer "B.Cu") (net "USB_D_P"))
 (segment (start 110.5 106.3825) (end 110.5 106.375) (width 0.15) (layer "F.Cu") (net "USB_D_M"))
 (segment (start 112.375 104.5) (end 112.5 104.5) (width 0.15) (layer "F.Cu") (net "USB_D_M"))
 (segment (start 107.25 110.19) (end 107.25 108.9) (width 0.15) (layer "F.Cu") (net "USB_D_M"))
 (segment (start 110.5 107.225) (end 110.5 107.2175) (width 0.15) (layer "F.Cu") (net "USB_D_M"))
 (segment (start 108.25 110.19) (end 108.25 108.9) (width 0.15) (layer "F.Cu") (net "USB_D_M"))
 (segment (start 110.825 108.3) (end 110.825 107.55) (width 0.15) (layer "F.Cu") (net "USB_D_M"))
 (segment (start 110.825 107.55) (end 110.5 107.225) (width 0.15) (layer "F.Cu") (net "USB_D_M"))
 (segment (start 110.825 107.55) (end 110.5 107.225) (width 0.15) (layer "F.Cu") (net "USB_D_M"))
 (segment (start 110.825 108.3) (end 110.825 107.55) (width 0.15) (layer "F.Cu") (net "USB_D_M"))
 (segment (start 110.5 106.375) (end 112.375 104.5) (width 0.15) (layer "F.Cu") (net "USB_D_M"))
 (segment (start 110.5 107.225) (end 110.5 107.2175) (width 0.15) (layer "F.Cu") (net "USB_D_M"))
 (segment (start 110.5 107.2175) (end 110.5 106.3825) (width 0.15) (layer "F.Cu") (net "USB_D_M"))
 (via (at 110.825 108.3) (size 0.45) (drill 0.2) (layers "F.Cu" "B.Cu") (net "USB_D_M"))
 (via (at 107.25 108.9) (size 0.45) (drill 0.2) (layers "F.Cu" "B.Cu") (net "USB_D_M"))
 (via (at 108.25 108.9) (size 0.45) (drill 0.2) (layers "F.Cu" "B.Cu") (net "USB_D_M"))
 (segment (start 107.55 108.825) (end 107.275 109.1) (width 0.15) (layer "B.Cu") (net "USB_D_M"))
 (segment (start 110.75 109.475) (end 110.75 108.375) (width 0.15) (layer "B.Cu") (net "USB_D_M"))
 (segment (start 107.275 108.925) (end 107.275 109.5) (width 0.15) (layer "B.Cu") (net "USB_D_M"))
 (segment (start 110.75 109.475) (end 110.75 108.375) (width 0.15) (layer "B.Cu") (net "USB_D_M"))
 (segment (start 107.275 109.1) (end 107.275 109.5) (width 0.15) (layer "B.Cu") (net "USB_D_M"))
 (segment (start 108.175 108.825) (end 107.55 108.825) (width 0.15) (layer "B.Cu") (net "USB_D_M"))
 (segment (start 110.125 110.1) (end 110.75 109.475) (width 0.15) (layer "B.Cu") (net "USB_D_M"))
 (segment (start 107.875 110.1) (end 110.125 110.1) (width 0.15) (layer "B.Cu") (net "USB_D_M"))
 (segment (start 108.25 108.9) (end 108.175 108.825) (width 0.15) (layer "B.Cu") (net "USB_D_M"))
 (segment (start 107.25 108.9) (end 107.275 108.925) (width 0.15) (layer "B.Cu") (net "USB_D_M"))
 (segment (start 110.75 108.375) (end 110.825 108.3) (width 0.15) (layer "B.Cu") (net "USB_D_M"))
 (segment (start 107.875 110.1) (end 110.125 110.1) (width 0.15) (layer "B.Cu") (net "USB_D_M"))
 (segment (start 107.275 109.5) (end 107.875 110.1) (width 0.15) (layer "B.Cu") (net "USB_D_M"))
 (segment (start 110.75 108.375) (end 110.825 108.3) (width 0.15) (layer "B.Cu") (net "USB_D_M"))
 (segment (start 110.125 110.1) (end 110.75 109.475) (width 0.15) (layer "B.Cu") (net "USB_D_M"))
 (segment (start 107.275 109.5) (end 107.875 110.1) (width 0.15) (layer "B.Cu") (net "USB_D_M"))
 (segment (start 109 107.2175) (end 109 106.3825) (width 0.15) (layer "F.Cu") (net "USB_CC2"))
 (segment (start 108.925 107.15) (end 109 107.225) (width 0.15) (layer "F.Cu") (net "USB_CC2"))
 (segment (start 109 104.6) (end 108.9 104.5) (width 0.15) (layer "F.Cu") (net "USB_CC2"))
 (segment (start 108.925 105.825) (end 108.925 107.15) (width 0.15) (layer "F.Cu") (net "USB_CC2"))
 (segment (start 109 107.225) (end 109 107.2175) (width 0.15) (layer "F.Cu") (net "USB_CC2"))
 (segment (start 109 106.3825) (end 109 106.375) (width 0.15) (layer "F.Cu") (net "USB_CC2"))
 (segment (start 109.75 110.19) (end 109.75 109.3) (width 0.15) (layer "F.Cu") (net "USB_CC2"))
 (segment (start 109 106.375) (end 109 104.6) (width 0.15) (layer "F.Cu") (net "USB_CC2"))
 (via (at 108.925 105.825) (size 0.45) (drill 0.2) (layers "F.Cu" "B.Cu") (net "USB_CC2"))
 (via (at 109.75 109.3) (size 0.45) (drill 0.2) (layers "F.Cu" "B.Cu") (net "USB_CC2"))
 (segment (start 109.75 106.65) (end 108.925 105.825) (width 0.15) (layer "B.Cu") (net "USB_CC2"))
 (segment (start 109.75 109.3) (end 109.75 106.65) (width 0.15) (layer "B.Cu") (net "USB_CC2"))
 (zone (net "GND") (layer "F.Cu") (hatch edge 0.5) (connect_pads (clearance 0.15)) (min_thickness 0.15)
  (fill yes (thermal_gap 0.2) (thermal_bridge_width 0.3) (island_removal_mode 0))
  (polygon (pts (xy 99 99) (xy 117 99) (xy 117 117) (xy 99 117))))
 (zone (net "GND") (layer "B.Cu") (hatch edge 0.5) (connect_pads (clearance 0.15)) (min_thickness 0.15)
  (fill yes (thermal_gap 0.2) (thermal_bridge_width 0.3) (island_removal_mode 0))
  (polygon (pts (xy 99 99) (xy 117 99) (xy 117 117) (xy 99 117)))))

